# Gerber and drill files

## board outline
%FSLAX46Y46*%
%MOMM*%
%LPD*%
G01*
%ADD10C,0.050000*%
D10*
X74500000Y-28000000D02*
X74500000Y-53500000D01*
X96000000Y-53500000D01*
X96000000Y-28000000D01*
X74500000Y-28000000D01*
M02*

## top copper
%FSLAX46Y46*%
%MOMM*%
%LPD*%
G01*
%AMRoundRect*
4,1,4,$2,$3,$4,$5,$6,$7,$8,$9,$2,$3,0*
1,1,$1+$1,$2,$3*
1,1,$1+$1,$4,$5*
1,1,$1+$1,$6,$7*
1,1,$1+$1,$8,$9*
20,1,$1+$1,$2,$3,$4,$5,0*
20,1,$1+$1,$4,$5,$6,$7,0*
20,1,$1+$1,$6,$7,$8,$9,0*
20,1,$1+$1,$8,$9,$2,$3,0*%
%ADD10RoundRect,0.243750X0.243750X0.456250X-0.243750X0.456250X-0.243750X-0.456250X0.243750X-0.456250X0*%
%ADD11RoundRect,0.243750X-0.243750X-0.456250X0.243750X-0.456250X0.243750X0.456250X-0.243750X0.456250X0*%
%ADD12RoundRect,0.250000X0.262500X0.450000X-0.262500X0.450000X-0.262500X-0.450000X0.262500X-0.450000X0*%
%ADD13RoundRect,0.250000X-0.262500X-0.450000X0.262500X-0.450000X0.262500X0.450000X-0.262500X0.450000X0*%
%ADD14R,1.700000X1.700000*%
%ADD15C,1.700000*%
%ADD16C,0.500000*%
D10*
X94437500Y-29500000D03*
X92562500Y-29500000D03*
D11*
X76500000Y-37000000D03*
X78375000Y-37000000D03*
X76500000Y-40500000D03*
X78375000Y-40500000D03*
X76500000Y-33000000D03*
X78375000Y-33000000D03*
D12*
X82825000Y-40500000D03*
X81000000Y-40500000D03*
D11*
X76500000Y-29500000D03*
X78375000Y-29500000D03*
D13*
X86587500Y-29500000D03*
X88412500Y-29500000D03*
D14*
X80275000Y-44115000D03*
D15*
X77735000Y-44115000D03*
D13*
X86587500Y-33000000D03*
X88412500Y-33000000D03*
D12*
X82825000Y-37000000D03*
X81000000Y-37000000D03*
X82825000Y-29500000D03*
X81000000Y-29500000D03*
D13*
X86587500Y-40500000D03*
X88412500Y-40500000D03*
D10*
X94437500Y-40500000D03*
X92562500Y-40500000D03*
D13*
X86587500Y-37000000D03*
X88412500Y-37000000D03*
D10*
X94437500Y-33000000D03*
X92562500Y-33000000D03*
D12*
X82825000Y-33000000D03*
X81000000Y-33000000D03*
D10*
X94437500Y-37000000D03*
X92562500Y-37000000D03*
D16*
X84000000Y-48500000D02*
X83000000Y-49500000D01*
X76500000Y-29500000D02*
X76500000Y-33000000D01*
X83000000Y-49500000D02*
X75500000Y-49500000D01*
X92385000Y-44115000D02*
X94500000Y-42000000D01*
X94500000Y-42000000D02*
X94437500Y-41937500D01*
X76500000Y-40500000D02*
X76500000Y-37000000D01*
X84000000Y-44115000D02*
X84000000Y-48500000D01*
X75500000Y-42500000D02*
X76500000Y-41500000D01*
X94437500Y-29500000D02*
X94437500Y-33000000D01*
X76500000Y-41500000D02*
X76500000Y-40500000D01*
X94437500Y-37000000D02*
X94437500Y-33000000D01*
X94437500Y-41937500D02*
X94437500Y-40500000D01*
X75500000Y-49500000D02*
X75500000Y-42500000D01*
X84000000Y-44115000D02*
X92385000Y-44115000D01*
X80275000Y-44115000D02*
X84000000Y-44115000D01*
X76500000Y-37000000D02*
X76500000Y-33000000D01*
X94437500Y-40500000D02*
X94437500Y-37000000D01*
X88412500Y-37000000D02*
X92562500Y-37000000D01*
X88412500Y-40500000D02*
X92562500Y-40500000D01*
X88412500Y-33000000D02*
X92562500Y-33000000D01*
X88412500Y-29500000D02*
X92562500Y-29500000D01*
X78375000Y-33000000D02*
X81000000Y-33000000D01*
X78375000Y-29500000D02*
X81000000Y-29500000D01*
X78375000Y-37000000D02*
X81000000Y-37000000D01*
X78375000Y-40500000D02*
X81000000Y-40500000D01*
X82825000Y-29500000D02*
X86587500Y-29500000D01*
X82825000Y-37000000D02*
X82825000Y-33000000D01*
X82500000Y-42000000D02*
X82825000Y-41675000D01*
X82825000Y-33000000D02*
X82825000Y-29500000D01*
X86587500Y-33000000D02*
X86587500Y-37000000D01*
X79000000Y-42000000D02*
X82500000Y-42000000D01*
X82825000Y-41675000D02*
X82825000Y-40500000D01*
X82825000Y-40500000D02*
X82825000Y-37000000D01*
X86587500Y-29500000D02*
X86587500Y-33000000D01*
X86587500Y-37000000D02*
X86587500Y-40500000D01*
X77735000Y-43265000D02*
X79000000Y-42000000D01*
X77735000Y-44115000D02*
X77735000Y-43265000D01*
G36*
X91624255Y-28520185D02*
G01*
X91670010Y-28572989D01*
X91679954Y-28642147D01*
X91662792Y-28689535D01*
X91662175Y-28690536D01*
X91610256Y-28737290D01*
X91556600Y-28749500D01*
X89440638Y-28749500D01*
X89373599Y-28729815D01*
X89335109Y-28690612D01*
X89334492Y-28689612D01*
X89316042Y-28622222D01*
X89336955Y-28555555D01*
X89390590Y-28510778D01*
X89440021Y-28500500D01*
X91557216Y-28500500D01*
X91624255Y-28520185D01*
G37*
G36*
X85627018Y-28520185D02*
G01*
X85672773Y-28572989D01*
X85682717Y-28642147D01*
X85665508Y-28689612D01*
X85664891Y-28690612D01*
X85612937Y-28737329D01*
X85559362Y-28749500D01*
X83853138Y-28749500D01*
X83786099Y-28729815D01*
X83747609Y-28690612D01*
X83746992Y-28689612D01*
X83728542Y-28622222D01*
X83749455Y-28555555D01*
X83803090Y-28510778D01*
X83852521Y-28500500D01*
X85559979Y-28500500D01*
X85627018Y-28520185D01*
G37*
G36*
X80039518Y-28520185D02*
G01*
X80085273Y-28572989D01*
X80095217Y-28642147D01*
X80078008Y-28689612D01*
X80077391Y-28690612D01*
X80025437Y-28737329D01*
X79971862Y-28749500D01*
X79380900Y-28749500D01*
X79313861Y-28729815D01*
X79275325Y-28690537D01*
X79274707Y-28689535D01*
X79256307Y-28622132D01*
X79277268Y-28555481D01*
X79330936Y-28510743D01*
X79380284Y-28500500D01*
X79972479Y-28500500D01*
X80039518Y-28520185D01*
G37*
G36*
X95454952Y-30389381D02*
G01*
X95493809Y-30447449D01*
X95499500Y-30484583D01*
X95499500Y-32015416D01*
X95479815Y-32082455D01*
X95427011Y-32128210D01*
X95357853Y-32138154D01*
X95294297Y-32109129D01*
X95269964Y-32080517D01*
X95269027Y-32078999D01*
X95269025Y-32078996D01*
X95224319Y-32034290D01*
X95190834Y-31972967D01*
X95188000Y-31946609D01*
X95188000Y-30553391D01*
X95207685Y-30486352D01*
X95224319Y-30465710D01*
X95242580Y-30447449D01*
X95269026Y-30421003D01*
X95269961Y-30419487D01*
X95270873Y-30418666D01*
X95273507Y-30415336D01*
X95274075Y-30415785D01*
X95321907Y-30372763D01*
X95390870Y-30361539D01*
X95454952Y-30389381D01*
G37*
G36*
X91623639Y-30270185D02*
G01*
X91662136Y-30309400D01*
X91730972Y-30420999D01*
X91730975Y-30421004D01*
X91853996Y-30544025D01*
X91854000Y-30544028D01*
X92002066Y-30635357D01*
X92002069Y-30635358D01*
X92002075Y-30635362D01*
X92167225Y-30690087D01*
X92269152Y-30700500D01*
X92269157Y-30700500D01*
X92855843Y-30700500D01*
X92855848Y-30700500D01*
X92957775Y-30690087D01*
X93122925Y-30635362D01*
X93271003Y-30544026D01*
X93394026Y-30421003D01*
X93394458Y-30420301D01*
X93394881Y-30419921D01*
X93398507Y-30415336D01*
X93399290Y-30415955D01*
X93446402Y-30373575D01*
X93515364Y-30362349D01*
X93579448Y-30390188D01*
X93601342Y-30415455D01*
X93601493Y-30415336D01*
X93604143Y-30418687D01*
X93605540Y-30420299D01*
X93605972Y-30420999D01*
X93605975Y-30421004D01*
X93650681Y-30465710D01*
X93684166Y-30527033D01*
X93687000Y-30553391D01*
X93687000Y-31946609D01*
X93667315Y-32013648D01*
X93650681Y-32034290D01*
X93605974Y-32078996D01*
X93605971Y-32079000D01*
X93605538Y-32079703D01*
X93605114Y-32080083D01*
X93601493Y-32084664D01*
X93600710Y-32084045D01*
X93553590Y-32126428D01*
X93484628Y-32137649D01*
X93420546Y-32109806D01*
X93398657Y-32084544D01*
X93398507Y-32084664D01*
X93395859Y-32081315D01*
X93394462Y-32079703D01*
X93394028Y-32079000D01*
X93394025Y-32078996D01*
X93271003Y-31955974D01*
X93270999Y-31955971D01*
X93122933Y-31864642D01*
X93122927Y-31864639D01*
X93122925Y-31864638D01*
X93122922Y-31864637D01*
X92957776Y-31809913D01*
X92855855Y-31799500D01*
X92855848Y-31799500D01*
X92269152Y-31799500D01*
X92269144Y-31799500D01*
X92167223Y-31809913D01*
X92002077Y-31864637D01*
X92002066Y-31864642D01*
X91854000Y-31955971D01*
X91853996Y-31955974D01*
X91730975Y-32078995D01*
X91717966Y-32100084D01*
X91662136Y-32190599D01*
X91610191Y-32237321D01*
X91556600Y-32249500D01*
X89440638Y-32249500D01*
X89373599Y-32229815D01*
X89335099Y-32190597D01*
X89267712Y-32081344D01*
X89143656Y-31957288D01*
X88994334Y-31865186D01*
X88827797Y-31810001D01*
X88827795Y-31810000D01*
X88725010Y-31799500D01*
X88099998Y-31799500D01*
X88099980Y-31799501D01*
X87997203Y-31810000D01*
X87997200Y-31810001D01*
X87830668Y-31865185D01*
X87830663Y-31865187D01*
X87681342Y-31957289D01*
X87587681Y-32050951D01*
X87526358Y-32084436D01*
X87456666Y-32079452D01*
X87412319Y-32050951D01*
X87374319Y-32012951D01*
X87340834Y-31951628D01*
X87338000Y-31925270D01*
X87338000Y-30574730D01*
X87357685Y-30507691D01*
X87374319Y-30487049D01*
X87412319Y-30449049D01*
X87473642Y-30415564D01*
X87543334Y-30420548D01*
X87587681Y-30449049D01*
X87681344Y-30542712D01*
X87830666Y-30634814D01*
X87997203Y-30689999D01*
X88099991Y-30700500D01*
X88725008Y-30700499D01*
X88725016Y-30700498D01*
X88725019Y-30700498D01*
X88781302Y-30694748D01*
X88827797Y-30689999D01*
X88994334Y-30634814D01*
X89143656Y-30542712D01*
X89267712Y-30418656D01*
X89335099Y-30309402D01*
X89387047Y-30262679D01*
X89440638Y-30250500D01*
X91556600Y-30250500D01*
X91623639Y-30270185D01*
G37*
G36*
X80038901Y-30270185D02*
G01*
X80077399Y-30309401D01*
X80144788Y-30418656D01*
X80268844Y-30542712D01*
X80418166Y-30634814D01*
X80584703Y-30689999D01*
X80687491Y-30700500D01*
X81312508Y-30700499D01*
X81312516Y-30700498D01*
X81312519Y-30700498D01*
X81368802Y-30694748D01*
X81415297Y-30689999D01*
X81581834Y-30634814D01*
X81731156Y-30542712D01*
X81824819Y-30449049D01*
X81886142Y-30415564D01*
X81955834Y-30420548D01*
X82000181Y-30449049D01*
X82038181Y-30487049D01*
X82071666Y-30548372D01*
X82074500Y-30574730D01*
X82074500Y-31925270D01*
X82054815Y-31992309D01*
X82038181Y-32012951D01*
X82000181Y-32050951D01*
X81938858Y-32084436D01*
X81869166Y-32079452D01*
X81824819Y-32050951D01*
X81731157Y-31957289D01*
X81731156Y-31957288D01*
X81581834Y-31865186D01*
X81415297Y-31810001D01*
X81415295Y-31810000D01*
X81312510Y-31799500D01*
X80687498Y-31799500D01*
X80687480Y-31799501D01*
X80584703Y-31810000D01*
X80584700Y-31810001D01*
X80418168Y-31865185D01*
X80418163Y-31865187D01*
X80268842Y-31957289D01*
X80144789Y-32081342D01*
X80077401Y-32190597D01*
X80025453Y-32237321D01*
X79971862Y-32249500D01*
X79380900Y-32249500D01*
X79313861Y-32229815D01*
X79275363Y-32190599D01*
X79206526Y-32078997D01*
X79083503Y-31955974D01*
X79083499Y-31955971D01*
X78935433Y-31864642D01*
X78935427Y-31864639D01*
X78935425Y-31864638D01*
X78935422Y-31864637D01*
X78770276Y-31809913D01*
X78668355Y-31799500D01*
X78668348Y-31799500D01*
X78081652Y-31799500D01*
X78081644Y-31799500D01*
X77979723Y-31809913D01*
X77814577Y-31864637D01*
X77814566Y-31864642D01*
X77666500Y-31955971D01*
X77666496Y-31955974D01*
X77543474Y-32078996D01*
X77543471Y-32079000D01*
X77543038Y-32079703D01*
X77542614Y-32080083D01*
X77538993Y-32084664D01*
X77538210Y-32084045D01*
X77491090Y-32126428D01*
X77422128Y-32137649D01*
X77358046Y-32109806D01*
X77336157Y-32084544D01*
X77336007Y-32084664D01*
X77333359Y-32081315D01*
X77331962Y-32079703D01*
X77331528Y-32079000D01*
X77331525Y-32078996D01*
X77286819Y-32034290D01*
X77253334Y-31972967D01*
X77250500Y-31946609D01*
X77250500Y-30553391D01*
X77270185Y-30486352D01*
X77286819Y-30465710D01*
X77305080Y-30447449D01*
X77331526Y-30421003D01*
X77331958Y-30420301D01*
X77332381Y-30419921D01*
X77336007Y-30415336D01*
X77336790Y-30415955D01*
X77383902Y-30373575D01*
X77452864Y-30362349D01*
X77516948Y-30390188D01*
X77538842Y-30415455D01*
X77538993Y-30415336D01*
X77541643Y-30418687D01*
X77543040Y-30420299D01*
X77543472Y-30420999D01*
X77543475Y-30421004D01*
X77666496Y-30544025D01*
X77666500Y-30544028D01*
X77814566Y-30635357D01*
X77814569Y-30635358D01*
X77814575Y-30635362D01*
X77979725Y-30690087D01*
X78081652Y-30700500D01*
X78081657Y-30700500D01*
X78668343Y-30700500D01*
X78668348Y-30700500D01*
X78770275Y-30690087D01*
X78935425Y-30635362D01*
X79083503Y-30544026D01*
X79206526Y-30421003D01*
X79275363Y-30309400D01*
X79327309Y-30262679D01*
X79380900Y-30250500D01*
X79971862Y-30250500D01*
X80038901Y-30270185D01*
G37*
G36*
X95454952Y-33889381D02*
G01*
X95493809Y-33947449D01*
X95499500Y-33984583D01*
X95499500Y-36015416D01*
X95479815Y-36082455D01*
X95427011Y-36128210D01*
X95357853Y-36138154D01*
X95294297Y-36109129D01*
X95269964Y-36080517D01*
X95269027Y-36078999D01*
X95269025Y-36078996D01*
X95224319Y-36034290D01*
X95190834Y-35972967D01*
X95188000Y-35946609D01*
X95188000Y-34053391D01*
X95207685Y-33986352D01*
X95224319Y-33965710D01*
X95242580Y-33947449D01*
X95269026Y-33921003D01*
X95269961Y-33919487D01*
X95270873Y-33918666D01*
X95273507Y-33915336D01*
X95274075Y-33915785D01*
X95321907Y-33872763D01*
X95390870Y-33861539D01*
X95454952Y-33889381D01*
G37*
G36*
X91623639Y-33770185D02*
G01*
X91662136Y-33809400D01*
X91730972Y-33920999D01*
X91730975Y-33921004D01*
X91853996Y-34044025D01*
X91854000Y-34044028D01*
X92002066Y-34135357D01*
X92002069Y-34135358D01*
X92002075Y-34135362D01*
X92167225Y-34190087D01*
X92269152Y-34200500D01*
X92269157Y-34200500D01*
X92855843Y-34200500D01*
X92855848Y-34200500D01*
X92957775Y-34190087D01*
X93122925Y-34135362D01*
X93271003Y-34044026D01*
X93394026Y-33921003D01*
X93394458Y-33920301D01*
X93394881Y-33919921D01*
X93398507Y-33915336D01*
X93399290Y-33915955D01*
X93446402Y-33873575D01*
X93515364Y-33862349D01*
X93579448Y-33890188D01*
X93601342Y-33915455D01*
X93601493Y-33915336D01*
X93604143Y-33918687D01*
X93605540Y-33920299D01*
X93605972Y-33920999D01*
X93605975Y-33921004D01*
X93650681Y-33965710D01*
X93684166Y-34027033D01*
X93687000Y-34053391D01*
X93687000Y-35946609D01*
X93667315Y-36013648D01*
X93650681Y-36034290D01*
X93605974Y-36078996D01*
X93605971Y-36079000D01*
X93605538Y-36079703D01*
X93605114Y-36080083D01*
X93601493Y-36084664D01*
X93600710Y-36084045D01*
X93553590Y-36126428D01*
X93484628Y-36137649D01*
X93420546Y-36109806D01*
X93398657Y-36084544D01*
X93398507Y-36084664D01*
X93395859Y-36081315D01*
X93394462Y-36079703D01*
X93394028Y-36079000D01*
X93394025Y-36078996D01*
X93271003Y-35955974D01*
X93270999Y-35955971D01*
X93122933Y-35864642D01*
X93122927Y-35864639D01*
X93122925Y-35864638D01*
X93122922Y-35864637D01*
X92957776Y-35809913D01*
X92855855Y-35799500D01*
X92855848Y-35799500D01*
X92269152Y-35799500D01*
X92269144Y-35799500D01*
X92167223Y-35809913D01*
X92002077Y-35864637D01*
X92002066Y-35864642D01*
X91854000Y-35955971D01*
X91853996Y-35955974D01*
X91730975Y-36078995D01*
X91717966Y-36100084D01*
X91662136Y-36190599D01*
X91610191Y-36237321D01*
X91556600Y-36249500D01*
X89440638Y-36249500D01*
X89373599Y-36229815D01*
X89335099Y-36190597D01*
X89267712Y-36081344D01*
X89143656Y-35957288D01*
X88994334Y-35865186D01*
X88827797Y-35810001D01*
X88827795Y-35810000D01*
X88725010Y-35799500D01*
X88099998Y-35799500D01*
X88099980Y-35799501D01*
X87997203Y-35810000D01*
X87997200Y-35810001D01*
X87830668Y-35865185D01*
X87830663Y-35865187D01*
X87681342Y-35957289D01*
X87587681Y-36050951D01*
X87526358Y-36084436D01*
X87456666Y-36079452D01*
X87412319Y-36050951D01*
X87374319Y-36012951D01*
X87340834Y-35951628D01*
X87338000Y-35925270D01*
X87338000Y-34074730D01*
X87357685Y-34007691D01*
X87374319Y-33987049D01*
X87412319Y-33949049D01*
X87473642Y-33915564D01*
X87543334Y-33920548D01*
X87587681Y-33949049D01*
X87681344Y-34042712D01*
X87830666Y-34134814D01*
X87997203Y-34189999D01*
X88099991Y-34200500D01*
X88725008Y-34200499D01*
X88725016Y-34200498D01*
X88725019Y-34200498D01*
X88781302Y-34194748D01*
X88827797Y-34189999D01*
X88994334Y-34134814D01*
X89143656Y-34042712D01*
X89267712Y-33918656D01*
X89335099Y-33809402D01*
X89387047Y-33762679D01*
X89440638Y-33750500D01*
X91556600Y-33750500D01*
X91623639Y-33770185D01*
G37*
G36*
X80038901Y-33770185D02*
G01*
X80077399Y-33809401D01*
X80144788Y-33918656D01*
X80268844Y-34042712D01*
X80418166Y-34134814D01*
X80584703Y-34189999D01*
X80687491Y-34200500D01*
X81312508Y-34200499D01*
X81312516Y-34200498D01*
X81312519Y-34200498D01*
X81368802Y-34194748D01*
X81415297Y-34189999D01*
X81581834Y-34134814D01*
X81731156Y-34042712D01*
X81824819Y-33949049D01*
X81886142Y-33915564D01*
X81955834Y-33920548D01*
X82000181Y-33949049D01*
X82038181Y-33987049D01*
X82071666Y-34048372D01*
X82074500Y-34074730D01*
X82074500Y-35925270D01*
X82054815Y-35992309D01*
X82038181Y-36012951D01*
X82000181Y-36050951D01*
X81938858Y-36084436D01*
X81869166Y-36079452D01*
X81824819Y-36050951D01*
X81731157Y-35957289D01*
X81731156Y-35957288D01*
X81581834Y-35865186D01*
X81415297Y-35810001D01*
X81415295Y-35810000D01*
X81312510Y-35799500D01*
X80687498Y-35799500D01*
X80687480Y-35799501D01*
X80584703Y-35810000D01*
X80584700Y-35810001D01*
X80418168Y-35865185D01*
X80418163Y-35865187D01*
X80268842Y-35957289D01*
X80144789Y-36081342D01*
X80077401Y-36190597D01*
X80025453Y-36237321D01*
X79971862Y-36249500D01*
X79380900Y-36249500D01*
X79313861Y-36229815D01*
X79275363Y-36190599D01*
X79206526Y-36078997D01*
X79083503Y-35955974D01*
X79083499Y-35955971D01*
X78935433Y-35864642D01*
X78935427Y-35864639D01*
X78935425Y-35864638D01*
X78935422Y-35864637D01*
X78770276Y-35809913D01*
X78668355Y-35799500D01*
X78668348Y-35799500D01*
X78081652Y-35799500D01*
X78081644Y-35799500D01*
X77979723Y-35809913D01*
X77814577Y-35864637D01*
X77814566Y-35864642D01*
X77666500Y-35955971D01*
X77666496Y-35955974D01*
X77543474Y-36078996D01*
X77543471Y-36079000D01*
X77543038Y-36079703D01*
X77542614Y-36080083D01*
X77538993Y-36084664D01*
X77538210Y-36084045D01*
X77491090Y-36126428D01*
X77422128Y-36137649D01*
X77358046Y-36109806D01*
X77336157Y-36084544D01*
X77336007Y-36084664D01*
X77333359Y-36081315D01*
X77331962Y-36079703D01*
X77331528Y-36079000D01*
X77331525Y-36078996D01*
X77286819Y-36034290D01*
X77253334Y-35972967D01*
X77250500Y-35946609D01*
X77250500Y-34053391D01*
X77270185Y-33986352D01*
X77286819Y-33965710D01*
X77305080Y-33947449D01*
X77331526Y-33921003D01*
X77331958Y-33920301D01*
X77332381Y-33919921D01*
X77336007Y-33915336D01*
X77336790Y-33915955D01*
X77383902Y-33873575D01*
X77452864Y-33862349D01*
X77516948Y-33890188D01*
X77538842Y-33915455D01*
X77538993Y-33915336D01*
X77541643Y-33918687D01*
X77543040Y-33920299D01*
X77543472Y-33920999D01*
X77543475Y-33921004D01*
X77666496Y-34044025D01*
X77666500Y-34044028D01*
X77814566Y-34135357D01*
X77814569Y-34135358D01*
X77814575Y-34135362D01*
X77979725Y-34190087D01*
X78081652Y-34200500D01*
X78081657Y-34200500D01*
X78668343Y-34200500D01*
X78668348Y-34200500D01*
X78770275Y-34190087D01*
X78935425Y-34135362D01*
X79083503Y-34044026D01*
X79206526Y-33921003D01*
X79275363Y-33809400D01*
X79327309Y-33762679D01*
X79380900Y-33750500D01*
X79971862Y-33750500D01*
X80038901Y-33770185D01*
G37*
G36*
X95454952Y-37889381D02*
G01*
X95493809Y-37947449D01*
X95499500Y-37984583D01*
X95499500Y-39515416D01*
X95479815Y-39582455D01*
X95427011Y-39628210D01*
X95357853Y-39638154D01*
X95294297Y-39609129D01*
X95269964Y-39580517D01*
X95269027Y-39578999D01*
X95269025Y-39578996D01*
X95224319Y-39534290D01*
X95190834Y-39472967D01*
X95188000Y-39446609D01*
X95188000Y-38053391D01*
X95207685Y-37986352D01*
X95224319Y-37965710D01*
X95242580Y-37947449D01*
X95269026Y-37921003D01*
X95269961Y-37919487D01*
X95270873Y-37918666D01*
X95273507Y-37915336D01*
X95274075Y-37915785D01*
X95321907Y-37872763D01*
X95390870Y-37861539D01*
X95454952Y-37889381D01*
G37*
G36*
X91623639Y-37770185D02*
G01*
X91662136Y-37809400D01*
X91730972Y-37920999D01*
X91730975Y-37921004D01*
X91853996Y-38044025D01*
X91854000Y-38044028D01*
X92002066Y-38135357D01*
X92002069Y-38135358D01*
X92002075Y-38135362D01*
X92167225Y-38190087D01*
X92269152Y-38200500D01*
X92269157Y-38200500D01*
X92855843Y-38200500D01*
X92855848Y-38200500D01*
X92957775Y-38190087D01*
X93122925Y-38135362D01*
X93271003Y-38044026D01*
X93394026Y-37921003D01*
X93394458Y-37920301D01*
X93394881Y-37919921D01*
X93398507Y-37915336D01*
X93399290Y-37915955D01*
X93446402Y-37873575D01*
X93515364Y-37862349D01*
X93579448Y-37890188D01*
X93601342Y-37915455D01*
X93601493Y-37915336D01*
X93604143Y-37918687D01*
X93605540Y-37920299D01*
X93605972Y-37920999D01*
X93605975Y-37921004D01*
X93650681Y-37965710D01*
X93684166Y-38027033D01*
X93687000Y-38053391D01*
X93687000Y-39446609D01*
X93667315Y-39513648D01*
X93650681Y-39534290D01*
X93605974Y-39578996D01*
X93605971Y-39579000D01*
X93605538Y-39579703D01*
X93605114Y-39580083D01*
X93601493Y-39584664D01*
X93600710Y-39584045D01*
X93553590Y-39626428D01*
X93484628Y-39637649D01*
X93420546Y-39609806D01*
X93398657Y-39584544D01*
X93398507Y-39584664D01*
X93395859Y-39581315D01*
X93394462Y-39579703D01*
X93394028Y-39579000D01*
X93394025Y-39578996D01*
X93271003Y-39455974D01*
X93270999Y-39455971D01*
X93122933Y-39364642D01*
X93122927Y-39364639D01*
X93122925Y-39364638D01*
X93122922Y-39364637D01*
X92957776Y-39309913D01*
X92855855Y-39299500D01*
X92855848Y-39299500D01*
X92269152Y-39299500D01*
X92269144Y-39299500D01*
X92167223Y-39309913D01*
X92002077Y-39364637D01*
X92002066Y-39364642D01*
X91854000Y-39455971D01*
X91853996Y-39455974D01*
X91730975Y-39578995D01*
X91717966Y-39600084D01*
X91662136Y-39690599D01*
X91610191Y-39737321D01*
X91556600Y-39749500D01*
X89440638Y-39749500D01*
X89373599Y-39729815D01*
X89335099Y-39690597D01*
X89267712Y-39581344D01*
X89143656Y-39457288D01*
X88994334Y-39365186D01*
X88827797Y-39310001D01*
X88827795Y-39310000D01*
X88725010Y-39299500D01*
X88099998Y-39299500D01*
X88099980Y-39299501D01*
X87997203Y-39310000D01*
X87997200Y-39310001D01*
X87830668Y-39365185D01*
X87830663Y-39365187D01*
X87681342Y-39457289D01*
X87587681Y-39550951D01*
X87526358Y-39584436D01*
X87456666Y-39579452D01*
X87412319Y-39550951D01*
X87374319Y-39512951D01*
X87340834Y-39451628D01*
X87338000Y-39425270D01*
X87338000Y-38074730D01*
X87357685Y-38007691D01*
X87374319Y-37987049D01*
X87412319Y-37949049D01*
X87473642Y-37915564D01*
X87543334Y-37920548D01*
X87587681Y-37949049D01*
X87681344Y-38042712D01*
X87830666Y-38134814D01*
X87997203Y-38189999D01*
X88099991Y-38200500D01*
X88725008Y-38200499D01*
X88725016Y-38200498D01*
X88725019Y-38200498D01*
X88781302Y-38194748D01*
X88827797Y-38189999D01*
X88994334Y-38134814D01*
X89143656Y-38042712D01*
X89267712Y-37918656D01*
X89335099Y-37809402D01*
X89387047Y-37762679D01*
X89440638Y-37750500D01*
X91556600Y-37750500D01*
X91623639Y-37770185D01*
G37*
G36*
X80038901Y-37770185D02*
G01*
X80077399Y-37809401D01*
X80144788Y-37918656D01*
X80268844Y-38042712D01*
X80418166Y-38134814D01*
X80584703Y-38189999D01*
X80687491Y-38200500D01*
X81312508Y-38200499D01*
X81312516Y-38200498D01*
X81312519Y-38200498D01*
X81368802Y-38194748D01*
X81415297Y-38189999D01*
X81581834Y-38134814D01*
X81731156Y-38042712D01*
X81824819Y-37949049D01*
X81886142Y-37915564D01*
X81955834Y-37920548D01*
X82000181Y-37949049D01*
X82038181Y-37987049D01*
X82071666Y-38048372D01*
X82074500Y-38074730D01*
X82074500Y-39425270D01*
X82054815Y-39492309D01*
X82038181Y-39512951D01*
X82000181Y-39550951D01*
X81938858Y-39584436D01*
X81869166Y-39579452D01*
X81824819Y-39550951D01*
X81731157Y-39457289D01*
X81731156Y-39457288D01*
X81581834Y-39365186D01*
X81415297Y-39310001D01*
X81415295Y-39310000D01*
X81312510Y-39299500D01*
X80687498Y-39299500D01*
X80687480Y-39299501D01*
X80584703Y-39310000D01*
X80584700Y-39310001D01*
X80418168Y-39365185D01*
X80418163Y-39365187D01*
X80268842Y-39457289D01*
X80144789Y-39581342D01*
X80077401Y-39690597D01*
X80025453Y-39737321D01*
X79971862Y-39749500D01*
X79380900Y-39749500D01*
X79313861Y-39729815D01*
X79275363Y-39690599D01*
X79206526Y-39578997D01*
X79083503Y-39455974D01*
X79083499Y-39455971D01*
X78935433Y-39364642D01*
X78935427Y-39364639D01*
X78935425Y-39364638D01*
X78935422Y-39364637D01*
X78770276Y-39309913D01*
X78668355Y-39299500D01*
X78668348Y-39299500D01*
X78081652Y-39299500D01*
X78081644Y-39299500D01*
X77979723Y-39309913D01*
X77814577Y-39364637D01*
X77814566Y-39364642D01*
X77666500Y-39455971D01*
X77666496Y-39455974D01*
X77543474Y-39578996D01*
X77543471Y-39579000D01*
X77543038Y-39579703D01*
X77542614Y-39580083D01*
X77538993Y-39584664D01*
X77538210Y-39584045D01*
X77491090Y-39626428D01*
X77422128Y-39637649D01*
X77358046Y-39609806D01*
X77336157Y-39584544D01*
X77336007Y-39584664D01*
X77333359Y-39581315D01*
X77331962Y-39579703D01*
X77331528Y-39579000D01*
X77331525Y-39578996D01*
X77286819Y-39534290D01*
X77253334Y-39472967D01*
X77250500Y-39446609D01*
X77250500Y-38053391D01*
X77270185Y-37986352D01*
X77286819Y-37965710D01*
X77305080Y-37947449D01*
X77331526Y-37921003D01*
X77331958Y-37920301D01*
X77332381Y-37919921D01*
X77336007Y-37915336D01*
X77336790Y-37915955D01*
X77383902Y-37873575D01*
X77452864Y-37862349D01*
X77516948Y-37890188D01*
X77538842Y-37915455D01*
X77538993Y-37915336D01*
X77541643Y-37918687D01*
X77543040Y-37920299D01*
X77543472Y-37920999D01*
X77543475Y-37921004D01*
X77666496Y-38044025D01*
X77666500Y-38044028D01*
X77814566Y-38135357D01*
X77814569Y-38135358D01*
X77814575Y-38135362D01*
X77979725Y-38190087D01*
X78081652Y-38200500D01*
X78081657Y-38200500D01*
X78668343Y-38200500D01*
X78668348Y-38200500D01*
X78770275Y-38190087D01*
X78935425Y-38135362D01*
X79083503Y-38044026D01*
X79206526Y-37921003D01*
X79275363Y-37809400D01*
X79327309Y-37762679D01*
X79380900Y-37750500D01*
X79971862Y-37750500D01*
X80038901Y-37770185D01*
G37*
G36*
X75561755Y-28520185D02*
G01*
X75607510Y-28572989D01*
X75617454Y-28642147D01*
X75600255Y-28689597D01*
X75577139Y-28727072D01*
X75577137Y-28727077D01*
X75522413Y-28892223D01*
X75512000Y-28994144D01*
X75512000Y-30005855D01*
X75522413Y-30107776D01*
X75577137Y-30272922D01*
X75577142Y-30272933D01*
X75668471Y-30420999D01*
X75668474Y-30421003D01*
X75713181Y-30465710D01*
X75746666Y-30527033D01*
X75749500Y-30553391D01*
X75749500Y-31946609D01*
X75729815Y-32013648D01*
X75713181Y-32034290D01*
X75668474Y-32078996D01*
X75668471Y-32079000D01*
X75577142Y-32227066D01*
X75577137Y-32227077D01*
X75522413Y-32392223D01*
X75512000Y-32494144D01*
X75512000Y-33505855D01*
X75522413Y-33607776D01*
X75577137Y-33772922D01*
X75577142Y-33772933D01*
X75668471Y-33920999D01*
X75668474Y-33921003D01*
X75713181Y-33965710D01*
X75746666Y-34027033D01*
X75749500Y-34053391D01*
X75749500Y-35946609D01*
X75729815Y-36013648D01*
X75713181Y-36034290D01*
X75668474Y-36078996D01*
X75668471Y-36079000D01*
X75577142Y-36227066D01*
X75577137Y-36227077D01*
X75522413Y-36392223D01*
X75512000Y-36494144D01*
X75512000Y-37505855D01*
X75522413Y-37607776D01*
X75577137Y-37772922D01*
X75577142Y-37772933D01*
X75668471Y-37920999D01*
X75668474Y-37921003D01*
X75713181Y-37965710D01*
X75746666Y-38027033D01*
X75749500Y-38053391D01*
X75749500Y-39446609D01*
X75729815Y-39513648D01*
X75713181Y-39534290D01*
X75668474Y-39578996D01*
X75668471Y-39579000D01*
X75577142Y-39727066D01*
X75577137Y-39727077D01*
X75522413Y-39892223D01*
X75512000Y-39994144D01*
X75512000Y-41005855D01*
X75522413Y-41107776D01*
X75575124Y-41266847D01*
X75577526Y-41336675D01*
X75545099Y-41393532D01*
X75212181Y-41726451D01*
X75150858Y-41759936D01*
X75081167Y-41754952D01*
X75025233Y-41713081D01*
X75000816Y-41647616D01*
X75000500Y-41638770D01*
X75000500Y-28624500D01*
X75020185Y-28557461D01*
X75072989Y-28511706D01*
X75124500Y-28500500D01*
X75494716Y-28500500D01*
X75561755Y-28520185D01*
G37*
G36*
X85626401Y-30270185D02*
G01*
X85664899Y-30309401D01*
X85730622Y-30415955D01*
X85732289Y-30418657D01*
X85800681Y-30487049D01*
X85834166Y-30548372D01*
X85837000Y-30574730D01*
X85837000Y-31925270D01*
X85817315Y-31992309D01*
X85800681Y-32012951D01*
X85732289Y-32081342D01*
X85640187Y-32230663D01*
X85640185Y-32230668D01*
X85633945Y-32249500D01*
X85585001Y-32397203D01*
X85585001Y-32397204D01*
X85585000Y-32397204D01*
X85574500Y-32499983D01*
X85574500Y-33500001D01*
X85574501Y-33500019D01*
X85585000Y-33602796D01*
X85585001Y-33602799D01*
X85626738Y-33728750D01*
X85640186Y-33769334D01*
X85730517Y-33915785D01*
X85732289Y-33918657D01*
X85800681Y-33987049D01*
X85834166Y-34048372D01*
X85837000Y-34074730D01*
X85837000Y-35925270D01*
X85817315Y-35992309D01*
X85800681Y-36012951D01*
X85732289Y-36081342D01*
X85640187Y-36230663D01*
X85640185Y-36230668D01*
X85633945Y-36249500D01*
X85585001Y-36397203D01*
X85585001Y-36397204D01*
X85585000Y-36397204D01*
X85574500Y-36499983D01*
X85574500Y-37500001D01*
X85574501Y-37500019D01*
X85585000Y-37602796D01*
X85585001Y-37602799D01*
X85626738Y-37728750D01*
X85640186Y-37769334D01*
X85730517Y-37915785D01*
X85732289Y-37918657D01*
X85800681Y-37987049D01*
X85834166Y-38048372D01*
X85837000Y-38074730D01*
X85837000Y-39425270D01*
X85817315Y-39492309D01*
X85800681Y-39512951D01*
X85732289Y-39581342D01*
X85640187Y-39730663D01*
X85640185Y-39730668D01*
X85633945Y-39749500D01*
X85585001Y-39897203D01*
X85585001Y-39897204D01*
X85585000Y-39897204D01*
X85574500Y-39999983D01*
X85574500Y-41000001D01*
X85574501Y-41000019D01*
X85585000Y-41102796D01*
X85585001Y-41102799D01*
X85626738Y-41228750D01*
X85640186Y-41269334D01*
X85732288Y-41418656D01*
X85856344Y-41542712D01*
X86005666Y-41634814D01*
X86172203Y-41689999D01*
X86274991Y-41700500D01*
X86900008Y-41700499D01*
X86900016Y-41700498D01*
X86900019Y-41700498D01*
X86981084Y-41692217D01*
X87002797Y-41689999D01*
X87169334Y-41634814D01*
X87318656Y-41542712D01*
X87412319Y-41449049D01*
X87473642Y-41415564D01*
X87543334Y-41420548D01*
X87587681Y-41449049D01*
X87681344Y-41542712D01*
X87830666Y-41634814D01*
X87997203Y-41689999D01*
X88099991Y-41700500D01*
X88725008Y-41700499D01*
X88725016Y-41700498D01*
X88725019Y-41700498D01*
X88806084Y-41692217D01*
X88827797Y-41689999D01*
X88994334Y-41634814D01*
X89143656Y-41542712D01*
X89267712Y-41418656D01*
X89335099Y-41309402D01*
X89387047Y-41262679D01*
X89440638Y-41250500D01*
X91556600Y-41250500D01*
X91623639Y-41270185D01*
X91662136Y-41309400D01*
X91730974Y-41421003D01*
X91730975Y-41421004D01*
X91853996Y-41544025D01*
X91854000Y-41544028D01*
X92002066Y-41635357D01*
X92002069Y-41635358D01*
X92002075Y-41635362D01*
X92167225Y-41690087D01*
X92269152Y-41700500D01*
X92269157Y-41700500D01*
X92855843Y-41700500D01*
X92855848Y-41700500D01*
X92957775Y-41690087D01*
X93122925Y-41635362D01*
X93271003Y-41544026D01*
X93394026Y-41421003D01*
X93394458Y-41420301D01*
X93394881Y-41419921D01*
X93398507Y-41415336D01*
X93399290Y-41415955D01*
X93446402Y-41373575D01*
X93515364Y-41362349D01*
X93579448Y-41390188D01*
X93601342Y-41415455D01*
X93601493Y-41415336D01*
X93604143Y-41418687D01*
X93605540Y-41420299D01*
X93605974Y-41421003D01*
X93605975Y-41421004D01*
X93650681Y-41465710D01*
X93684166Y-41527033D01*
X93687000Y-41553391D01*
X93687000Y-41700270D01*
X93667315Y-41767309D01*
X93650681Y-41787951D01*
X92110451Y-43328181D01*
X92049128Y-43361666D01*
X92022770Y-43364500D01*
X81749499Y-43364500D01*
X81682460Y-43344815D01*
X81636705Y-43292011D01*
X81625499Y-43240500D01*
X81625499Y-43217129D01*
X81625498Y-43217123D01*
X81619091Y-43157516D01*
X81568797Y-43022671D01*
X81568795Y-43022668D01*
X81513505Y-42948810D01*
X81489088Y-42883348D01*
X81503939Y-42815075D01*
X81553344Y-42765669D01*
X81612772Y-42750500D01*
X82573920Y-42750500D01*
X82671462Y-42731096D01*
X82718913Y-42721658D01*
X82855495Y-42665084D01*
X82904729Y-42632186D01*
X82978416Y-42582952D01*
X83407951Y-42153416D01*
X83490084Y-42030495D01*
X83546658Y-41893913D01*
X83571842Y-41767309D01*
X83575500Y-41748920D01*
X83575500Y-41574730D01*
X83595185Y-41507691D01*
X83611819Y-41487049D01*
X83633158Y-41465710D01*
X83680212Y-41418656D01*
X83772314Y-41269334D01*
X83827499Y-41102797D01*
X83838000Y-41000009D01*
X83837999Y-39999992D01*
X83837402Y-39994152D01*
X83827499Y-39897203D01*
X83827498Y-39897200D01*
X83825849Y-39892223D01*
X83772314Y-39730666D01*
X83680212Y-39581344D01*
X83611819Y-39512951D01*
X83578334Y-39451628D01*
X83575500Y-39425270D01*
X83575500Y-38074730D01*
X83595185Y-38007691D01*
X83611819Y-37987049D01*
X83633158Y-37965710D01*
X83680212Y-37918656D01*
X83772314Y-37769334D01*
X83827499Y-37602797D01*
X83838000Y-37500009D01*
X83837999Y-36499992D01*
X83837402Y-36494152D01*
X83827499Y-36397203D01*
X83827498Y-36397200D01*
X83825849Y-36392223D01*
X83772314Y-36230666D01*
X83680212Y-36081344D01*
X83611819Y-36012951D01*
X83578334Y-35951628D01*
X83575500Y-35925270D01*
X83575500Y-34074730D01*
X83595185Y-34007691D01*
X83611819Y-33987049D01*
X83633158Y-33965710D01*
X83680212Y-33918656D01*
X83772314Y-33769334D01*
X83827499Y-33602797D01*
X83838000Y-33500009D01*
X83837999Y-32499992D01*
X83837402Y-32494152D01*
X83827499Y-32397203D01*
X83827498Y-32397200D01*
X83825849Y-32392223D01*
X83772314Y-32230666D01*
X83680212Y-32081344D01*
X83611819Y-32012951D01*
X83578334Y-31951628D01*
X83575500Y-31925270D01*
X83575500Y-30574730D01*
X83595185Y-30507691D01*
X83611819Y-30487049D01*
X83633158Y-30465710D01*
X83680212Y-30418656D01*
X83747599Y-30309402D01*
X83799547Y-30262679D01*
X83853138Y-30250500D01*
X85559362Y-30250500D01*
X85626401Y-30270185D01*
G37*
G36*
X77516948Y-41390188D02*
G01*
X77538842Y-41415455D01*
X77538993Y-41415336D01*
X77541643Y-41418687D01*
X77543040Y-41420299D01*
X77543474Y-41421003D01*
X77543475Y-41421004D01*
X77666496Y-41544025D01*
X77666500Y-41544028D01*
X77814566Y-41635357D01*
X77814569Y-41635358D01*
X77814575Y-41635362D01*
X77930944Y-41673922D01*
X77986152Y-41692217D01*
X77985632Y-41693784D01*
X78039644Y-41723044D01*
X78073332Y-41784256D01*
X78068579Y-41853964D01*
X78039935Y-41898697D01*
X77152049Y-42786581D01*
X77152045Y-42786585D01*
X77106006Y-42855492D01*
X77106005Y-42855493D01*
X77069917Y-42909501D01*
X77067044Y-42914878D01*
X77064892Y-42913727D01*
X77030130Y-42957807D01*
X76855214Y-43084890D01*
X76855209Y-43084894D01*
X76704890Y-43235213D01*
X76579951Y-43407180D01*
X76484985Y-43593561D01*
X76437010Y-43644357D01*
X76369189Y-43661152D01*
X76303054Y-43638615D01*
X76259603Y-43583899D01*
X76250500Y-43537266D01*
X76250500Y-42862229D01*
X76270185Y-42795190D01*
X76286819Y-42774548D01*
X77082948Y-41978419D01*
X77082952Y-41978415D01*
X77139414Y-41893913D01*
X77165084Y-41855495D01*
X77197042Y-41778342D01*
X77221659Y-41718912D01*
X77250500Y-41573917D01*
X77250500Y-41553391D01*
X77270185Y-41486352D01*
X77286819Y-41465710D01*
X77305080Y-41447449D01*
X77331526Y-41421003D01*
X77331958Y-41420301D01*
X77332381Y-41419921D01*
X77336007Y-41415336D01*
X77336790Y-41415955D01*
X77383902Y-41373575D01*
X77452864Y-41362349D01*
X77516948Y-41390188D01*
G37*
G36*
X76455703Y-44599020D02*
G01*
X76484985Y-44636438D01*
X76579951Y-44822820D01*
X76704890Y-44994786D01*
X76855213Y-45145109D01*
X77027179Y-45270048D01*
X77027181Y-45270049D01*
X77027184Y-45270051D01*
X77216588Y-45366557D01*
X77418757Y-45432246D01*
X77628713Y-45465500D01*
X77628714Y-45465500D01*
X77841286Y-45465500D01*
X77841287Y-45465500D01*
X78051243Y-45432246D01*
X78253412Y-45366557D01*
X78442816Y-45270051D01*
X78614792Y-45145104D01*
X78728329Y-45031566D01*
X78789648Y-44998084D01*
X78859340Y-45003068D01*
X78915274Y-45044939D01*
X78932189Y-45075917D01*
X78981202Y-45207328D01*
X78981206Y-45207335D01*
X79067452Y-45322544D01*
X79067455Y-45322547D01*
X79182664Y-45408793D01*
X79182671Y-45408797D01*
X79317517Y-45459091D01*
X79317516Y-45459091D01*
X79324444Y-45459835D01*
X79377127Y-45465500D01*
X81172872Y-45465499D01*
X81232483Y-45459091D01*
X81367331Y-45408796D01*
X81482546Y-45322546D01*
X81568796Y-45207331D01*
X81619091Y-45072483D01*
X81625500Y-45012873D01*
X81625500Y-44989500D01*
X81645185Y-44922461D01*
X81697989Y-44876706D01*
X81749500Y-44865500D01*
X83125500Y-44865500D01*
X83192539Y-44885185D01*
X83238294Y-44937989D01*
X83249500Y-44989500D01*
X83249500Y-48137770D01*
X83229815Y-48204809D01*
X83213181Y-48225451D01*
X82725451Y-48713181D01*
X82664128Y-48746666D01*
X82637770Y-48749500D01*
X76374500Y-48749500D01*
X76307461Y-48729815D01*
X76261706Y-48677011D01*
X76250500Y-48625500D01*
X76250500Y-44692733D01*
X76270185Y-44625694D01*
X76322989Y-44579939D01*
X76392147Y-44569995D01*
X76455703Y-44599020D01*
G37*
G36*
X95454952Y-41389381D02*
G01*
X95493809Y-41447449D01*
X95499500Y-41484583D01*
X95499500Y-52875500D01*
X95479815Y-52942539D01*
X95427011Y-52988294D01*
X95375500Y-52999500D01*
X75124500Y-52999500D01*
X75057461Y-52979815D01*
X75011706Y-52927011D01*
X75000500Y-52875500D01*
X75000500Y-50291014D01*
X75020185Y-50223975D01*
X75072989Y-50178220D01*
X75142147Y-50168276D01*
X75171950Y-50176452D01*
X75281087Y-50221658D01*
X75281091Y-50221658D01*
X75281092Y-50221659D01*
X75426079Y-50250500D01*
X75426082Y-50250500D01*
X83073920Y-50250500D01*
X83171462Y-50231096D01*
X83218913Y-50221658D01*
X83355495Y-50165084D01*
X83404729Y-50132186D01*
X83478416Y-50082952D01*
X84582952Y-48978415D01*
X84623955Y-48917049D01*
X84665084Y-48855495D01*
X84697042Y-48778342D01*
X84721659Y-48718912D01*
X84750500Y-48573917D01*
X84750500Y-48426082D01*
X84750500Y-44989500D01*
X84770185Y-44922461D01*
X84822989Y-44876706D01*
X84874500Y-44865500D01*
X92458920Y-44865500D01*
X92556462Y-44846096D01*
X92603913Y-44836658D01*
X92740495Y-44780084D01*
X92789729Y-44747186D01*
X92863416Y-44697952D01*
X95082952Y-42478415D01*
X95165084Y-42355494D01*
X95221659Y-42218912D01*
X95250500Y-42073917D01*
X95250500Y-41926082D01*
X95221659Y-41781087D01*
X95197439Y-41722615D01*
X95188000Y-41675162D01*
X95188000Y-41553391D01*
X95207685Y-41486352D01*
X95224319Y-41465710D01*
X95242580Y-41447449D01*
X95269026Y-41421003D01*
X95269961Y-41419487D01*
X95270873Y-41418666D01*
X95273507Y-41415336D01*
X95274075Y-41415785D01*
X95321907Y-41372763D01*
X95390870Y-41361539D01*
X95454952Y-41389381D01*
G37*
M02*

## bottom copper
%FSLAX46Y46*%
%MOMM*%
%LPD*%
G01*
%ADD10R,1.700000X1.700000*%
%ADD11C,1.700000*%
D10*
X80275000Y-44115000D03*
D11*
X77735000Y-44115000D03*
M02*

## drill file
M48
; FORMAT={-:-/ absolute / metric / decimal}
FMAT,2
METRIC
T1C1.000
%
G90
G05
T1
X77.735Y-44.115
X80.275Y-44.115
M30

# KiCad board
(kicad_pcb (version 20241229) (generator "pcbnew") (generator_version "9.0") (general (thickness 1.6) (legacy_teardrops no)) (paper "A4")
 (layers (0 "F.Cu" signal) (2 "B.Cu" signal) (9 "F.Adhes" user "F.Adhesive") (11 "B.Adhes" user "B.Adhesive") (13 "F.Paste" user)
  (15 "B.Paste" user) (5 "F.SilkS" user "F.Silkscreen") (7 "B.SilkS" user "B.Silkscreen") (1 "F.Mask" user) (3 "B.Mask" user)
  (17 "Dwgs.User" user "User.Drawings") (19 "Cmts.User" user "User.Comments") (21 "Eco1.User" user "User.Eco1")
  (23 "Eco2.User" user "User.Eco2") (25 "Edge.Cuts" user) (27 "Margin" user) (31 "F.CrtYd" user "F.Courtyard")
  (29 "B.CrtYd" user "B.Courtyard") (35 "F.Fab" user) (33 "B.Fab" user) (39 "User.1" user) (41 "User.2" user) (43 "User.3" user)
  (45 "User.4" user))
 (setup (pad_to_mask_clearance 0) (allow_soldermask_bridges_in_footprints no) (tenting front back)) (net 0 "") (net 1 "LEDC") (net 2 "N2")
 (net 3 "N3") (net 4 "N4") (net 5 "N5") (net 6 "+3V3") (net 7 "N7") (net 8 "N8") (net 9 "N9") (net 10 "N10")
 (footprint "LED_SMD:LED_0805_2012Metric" (layer "F.Cu") (at 93.5 29.5 180)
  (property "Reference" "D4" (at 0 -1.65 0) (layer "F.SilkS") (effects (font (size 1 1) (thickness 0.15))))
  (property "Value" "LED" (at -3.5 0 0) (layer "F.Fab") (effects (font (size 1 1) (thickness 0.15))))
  (pad "1" smd roundrect (at -0.9375 0 180) (size 0.975 1.4) (layers "F.Cu" "F.Mask" "F.Paste") (roundrect_rratio 0.25) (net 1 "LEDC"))
  (pad "2" smd roundrect (at 0.9375 0 180) (size 0.975 1.4) (layers "F.Cu" "F.Mask" "F.Paste") (roundrect_rratio 0.25) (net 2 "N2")))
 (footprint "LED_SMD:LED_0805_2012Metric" (layer "F.Cu") (at 77.4375 37)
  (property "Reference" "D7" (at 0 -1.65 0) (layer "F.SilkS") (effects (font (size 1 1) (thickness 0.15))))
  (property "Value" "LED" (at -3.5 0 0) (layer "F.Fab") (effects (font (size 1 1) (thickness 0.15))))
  (pad "1" smd roundrect (at -0.9375 0) (size 0.975 1.4) (layers "F.Cu" "F.Mask" "F.Paste") (roundrect_rratio 0.25) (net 1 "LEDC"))
  (pad "2" smd roundrect (at 0.9375 0) (size 0.975 1.4) (layers "F.Cu" "F.Mask" "F.Paste") (roundrect_rratio 0.25) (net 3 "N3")))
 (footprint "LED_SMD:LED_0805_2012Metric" (layer "F.Cu") (at 77.4375 40.5)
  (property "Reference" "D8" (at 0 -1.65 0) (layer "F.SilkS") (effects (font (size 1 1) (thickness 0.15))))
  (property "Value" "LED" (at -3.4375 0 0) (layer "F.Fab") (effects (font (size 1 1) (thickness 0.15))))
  (pad "1" smd roundrect (at -0.9375 0) (size 0.975 1.4) (layers "F.Cu" "F.Mask" "F.Paste") (roundrect_rratio 0.25) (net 1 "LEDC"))
  (pad "2" smd roundrect (at 0.9375 0) (size 0.975 1.4) (layers "F.Cu" "F.Mask" "F.Paste") (roundrect_rratio 0.25) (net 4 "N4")))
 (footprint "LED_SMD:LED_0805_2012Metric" (layer "F.Cu") (at 77.4375 33)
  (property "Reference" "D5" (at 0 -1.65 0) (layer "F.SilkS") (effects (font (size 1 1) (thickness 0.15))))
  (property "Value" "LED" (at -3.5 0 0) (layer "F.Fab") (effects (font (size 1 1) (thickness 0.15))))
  (pad "1" smd roundrect (at -0.9375 0) (size 0.975 1.4) (layers "F.Cu" "F.Mask" "F.Paste") (roundrect_rratio 0.25) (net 1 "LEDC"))
  (pad "2" smd roundrect (at 0.9375 0) (size 0.975 1.4) (layers "F.Cu" "F.Mask" "F.Paste") (roundrect_rratio 0.25) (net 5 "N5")))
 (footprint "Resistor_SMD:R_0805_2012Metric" (layer "F.Cu") (at 81.9125 40.5 180)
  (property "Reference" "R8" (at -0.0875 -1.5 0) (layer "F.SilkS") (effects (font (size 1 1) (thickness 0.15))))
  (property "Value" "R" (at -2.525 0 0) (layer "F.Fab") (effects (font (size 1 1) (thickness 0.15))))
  (pad "1" smd roundrect (at -0.9125 0 180) (size 1.025 1.4) (layers "F.Cu" "F.Mask" "F.Paste") (roundrect_rratio 0.243902) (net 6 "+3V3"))
  (pad "2" smd roundrect (at 0.9125 0 180) (size 1.025 1.4) (layers "F.Cu" "F.Mask" "F.Paste") (roundrect_rratio 0.243902) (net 4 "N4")))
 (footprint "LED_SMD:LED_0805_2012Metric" (layer "F.Cu") (at 77.4375 29.5)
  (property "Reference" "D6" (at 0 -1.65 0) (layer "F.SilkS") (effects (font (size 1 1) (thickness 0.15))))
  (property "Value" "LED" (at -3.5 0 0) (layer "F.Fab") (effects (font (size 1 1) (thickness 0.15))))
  (pad "1" smd roundrect (at -0.9375 0) (size 0.975 1.4) (layers "F.Cu" "F.Mask" "F.Paste") (roundrect_rratio 0.25) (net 1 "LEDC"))
  (pad "2" smd roundrect (at 0.9375 0) (size 0.975 1.4) (layers "F.Cu" "F.Mask" "F.Paste") (roundrect_rratio 0.25) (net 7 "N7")))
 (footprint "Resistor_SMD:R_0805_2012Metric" (layer "F.Cu") (at 87.5 29.5)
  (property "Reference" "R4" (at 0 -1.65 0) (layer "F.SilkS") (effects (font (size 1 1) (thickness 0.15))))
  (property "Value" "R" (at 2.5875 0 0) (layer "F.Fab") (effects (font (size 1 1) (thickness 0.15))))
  (pad "1" smd roundrect (at -0.9125 0) (size 1.025 1.4) (layers "F.Cu" "F.Mask" "F.Paste") (roundrect_rratio 0.243902) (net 6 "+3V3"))
  (pad "2" smd roundrect (at 0.9125 0) (size 1.025 1.4) (layers "F.Cu" "F.Mask" "F.Paste") (roundrect_rratio 0.243902) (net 2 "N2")))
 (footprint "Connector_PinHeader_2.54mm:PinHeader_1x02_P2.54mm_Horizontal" (layer "F.Cu") (at 80.275 44.115 -90)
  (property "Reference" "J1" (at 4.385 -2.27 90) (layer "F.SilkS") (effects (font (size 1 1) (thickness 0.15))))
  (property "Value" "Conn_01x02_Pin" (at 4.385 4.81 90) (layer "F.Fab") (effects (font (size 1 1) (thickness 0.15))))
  (pad "1" thru_hole rect (at 0 0 270) (size 1.7 1.7) (drill 1) (layers "*.Cu" "*.Mask") (remove_unused_layers no) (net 1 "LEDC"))
  (pad "2" thru_hole circle (at 0 2.54 270) (size 1.7 1.7) (drill 1) (layers "*.Cu" "*.Mask") (remove_unused_layers no) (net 6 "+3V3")))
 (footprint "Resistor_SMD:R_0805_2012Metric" (layer "F.Cu") (at 87.5 33)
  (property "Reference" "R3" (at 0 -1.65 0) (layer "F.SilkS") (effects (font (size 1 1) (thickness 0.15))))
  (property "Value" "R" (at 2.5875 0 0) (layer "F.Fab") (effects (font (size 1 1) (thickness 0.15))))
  (pad "1" smd roundrect (at -0.9125 0) (size 1.025 1.4) (layers "F.Cu" "F.Mask" "F.Paste") (roundrect_rratio 0.243902) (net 6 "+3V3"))
  (pad "2" smd roundrect (at 0.9125 0) (size 1.025 1.4) (layers "F.Cu" "F.Mask" "F.Paste") (roundrect_rratio 0.243902) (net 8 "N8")))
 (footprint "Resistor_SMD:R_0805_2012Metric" (layer "F.Cu") (at 81.9125 37 180)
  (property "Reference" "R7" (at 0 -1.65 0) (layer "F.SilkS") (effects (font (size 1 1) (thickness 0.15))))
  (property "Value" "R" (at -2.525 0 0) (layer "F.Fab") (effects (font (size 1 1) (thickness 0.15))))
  (pad "1" smd roundrect (at -0.9125 0 180) (size 1.025 1.4) (layers "F.Cu" "F.Mask" "F.Paste") (roundrect_rratio 0.243902) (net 6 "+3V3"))
  (pad "2" smd roundrect (at 0.9125 0 180) (size 1.025 1.4) (layers "F.Cu" "F.Mask" "F.Paste") (roundrect_rratio 0.243902) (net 3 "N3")))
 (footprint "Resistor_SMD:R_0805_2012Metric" (layer "F.Cu") (at 81.9125 29.5 180)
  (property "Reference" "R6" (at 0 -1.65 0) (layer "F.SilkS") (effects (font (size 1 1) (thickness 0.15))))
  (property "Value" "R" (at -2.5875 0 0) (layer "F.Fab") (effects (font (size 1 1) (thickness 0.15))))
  (pad "1" smd roundrect (at -0.9125 0 180) (size 1.025 1.4) (layers "F.Cu" "F.Mask" "F.Paste") (roundrect_rratio 0.243902) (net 6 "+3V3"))
  (pad "2" smd roundrect (at 0.9125 0 180) (size 1.025 1.4) (layers "F.Cu" "F.Mask" "F.Paste") (roundrect_rratio 0.243902) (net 7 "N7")))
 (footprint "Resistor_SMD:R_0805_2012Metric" (layer "F.Cu") (at 87.5 40.5)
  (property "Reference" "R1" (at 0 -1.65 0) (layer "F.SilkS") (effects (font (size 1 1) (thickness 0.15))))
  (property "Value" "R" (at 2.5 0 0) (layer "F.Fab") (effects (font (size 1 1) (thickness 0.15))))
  (pad "1" smd roundrect (at -0.9125 0) (size 1.025 1.4) (layers "F.Cu" "F.Mask" "F.Paste") (roundrect_rratio 0.243902) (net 6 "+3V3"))
  (pad "2" smd roundrect (at 0.9125 0) (size 1.025 1.4) (layers "F.Cu" "F.Mask" "F.Paste") (roundrect_rratio 0.243902) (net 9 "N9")))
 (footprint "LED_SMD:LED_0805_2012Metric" (layer "F.Cu") (at 93.5 40.5 180)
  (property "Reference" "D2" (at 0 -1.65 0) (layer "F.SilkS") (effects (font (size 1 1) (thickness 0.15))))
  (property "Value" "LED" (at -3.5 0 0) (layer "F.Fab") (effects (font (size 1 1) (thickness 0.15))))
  (pad "1" smd roundrect (at -0.9375 0 180) (size 0.975 1.4) (layers "F.Cu" "F.Mask" "F.Paste") (roundrect_rratio 0.25) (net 1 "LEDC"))
  (pad "2" smd roundrect (at 0.9375 0 180) (size 0.975 1.4) (layers "F.Cu" "F.Mask" "F.Paste") (roundrect_rratio 0.25) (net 9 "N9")))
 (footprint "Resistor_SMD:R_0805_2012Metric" (layer "F.Cu") (at 87.5 37)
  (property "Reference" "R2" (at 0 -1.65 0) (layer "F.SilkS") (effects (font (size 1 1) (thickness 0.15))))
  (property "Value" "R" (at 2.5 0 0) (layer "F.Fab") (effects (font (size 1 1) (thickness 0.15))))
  (pad "1" smd roundrect (at -0.9125 0) (size 1.025 1.4) (layers "F.Cu" "F.Mask" "F.Paste") (roundrect_rratio 0.243902) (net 6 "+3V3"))
  (pad "2" smd roundrect (at 0.9125 0) (size 1.025 1.4) (layers "F.Cu" "F.Mask" "F.Paste") (roundrect_rratio 0.243902) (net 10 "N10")))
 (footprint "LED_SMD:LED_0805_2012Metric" (layer "F.Cu") (at 93.5 33 180)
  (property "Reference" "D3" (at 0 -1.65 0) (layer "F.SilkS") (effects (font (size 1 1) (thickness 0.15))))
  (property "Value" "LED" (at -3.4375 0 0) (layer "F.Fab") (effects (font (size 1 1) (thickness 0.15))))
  (pad "1" smd roundrect (at -0.9375 0 180) (size 0.975 1.4) (layers "F.Cu" "F.Mask" "F.Paste") (roundrect_rratio 0.25) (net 1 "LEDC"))
  (pad "2" smd roundrect (at 0.9375 0 180) (size 0.975 1.4) (layers "F.Cu" "F.Mask" "F.Paste") (roundrect_rratio 0.25) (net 8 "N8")))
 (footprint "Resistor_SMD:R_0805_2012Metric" (layer "F.Cu") (at 81.9125 33 180)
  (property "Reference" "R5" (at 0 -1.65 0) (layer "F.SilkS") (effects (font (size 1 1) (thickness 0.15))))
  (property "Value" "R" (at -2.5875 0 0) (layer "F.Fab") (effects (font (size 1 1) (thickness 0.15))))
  (pad "1" smd roundrect (at -0.9125 0 180) (size 1.025 1.4) (layers "F.Cu" "F.Mask" "F.Paste") (roundrect_rratio 0.243902) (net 6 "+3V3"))
  (pad "2" smd roundrect (at 0.9125 0 180) (size 1.025 1.4) (layers "F.Cu" "F.Mask" "F.Paste") (roundrect_rratio 0.243902) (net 5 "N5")))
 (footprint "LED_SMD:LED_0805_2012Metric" (layer "F.Cu") (at 93.5 37 180)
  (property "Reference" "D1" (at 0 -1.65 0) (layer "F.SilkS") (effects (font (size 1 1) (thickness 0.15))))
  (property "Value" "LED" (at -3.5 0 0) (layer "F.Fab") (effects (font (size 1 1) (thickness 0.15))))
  (pad "1" smd roundrect (at -0.9375 0 180) (size 0.975 1.4) (layers "F.Cu" "F.Mask" "F.Paste") (roundrect_rratio 0.25) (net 1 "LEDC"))
  (pad "2" smd roundrect (at 0.9375 0 180) (size 0.975 1.4) (layers "F.Cu" "F.Mask" "F.Paste") (roundrect_rratio 0.25) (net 10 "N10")))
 (gr_poly (pts (xy 74.5 28) (xy 74.5 53.5) (xy 96 53.5) (xy 96 28)) (stroke (width 0.05) (type solid)) (fill no) (layer "Edge.Cuts"))
 (segment (start 84 48.5) (end 83 49.5) (width 0.5) (layer "F.Cu") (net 1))
 (segment (start 76.5 29.5) (end 76.5 33) (width 0.5) (layer "F.Cu") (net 1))
 (segment (start 83 49.5) (end 75.5 49.5) (width 0.5) (layer "F.Cu") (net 1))
 (segment (start 92.385 44.115) (end 94.5 42) (width 0.5) (layer "F.Cu") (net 1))
 (segment (start 94.5 42) (end 94.4375 41.9375) (width 0.5) (layer "F.Cu") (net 1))
 (segment (start 76.5 40.5) (end 76.5 37) (width 0.5) (layer "F.Cu") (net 1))
 (segment (start 84 44.115) (end 84 48.5) (width 0.5) (layer "F.Cu") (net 1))
 (segment (start 75.5 42.5) (end 76.5 41.5) (width 0.5) (layer "F.Cu") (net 1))
 (segment (start 94.4375 29.5) (end 94.4375 33) (width 0.5) (layer "F.Cu") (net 1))
 (segment (start 76.5 41.5) (end 76.5 40.5) (width 0.5) (layer "F.Cu") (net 1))
 (segment (start 94.4375 37) (end 94.4375 33) (width 0.5) (layer "F.Cu") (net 1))
 (segment (start 94.4375 41.9375) (end 94.4375 40.5) (width 0.5) (layer "F.Cu") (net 1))
 (segment (start 75.5 49.5) (end 75.5 42.5) (width 0.5) (layer "F.Cu") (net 1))
 (segment (start 84 44.115) (end 92.385 44.115) (width 0.5) (layer "F.Cu") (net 1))
 (segment (start 80.275 44.115) (end 84 44.115) (width 0.5) (layer "F.Cu") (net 1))
 (segment (start 76.5 37) (end 76.5 33) (width 0.5) (layer "F.Cu") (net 1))
 (segment (start 94.4375 40.5) (end 94.4375 37) (width 0.5) (layer "F.Cu") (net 1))
 (segment (start 88.4125 37) (end 92.5625 37) (width 0.5) (layer "F.Cu") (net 10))
 (segment (start 88.4125 40.5) (end 92.5625 40.5) (width 0.5) (layer "F.Cu") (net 9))
 (segment (start 88.4125 33) (end 92.5625 33) (width 0.5) (layer "F.Cu") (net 8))
 (segment (start 88.4125 29.5) (end 92.5625 29.5) (width 0.5) (layer "F.Cu") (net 2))
 (segment (start 78.375 33) (end 81 33) (width 0.5) (layer "F.Cu") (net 5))
 (segment (start 78.375 29.5) (end 81 29.5) (width 0.5) (layer "F.Cu") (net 7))
 (segment (start 78.375 37) (end 81 37) (width 0.5) (layer "F.Cu") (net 3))
 (segment (start 78.375 40.5) (end 81 40.5) (width 0.5) (layer "F.Cu") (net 4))
 (segment (start 82.825 29.5) (end 86.5875 29.5) (width 0.5) (layer "F.Cu") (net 6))
 (segment (start 82.825 37) (end 82.825 33) (width 0.5) (layer "F.Cu") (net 6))
 (segment (start 82.5 42) (end 82.825 41.675) (width 0.5) (layer "F.Cu") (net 6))
 (segment (start 82.825 33) (end 82.825 29.5) (width 0.5) (layer "F.Cu") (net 6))
 (segment (start 86.5875 33) (end 86.5875 37) (width 0.5) (layer "F.Cu") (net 6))
 (segment (start 79 42) (end 82.5 42) (width 0.5) (layer "F.Cu") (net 6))
 (segment (start 82.825 41.675) (end 82.825 40.5) (width 0.5) (layer "F.Cu") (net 6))
 (segment (start 82.825 40.5) (end 82.825 37) (width 0.5) (layer "F.Cu") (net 6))
 (segment (start 86.5875 29.5) (end 86.5875 33) (width 0.5) (layer "F.Cu") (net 6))
 (segment (start 86.5875 37) (end 86.5875 40.5) (width 0.5) (layer "F.Cu") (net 6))
 (segment (start 77.735 43.265) (end 79 42) (width 0.5) (layer "F.Cu") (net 6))
 (segment (start 77.735 44.115) (end 77.735 43.265) (width 0.5) (layer "F.Cu") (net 6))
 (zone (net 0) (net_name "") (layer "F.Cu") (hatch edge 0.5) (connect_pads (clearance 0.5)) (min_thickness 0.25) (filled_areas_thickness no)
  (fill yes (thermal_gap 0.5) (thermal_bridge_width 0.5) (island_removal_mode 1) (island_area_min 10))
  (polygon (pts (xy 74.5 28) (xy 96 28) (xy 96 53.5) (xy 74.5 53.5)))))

